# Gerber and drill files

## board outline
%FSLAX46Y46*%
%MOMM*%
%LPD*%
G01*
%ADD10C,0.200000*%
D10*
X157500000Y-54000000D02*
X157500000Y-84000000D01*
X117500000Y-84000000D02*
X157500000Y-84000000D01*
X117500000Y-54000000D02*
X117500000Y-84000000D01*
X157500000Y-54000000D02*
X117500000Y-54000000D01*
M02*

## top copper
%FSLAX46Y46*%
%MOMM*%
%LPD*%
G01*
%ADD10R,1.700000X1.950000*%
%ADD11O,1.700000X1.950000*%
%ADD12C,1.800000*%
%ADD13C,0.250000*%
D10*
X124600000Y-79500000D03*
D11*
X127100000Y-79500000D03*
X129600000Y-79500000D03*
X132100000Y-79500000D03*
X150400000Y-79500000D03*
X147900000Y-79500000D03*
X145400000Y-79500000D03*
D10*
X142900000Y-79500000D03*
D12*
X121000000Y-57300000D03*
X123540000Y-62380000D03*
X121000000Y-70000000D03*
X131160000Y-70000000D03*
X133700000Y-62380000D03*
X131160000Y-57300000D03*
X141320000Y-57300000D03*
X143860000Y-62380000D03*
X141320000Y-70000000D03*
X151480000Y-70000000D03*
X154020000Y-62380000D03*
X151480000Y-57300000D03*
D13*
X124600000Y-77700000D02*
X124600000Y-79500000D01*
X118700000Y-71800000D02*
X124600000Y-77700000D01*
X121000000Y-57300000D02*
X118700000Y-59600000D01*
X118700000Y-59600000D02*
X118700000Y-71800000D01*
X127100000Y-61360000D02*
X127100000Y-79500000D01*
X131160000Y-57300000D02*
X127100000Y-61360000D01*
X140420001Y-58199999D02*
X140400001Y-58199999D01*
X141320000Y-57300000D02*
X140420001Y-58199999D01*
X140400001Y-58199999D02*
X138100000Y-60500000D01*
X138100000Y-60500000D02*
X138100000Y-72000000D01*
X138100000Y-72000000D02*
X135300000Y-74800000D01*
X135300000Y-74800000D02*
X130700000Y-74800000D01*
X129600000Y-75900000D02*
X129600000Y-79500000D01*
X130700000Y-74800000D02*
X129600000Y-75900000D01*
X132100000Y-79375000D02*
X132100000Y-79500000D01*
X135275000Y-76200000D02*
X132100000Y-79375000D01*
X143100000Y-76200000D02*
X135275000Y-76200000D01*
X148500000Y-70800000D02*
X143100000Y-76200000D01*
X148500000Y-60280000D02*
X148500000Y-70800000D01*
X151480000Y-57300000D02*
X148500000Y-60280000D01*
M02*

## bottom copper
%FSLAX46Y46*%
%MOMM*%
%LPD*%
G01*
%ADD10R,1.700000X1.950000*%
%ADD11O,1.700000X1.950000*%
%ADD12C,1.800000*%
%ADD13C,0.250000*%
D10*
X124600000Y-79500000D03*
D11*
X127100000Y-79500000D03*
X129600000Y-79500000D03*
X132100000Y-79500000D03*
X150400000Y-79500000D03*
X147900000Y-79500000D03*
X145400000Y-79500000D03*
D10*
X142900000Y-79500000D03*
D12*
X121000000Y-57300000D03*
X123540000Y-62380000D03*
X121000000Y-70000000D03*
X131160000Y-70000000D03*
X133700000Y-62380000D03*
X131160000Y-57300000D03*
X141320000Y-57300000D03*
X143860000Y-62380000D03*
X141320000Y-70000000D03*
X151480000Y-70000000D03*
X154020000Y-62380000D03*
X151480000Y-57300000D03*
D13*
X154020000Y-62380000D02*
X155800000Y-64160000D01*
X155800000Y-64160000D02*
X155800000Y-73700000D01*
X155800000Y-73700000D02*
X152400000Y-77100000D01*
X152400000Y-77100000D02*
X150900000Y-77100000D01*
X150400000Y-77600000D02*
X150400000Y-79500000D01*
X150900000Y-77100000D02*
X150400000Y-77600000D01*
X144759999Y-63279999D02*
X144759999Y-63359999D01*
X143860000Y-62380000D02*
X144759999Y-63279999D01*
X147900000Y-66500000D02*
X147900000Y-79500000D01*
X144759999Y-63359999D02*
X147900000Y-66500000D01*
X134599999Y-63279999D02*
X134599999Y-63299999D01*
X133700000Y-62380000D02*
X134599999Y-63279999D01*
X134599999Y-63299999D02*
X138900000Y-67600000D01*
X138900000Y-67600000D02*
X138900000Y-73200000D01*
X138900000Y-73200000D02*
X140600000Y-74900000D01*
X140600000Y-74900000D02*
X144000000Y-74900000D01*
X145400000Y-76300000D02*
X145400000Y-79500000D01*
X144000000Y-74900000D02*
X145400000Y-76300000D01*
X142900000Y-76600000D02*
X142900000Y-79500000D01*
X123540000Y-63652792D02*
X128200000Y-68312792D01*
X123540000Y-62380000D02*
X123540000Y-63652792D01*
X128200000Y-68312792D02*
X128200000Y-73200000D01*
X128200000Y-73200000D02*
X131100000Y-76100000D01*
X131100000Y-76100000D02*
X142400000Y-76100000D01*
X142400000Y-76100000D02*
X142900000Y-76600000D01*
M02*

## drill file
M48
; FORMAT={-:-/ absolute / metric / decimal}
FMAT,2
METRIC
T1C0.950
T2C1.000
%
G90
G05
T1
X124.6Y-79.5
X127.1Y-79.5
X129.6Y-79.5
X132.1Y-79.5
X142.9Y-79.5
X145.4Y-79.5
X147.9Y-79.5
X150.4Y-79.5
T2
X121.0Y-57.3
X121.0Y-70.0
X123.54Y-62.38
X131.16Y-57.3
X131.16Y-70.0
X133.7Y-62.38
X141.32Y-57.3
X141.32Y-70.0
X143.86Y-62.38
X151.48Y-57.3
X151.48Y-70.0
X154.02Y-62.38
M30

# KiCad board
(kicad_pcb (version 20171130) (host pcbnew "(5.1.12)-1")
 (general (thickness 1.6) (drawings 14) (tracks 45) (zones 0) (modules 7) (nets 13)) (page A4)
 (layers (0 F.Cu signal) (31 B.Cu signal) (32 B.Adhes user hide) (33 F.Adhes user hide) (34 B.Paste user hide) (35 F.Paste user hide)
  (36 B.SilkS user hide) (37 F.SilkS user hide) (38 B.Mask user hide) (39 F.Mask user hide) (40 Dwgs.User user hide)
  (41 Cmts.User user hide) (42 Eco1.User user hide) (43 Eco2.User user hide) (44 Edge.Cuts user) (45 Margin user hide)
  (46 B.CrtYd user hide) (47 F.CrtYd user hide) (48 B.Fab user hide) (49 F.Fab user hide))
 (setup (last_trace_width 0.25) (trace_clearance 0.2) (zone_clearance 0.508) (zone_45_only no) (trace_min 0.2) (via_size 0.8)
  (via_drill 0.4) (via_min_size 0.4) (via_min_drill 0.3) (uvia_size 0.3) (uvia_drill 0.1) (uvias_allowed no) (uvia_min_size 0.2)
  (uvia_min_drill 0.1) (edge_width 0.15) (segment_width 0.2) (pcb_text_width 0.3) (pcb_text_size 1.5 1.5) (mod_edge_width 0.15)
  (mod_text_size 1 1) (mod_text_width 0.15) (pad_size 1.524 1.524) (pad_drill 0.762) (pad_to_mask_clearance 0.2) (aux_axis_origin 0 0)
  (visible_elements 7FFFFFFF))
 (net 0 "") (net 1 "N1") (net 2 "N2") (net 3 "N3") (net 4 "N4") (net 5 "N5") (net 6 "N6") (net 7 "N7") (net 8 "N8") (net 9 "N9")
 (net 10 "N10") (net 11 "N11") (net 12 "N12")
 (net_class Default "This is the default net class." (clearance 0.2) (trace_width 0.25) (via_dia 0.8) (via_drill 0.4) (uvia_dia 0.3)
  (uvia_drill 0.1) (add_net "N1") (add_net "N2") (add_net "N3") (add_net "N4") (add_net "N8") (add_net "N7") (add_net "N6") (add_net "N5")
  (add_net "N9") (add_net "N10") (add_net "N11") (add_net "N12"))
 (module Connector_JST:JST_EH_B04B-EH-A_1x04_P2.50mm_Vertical (layer F.Cu) (at 124.6 79.5)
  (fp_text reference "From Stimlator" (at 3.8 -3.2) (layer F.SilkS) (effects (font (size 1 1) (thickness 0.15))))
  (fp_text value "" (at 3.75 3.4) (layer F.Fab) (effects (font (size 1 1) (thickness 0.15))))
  (pad 1 thru_hole rect (at 0 0) (size 1.7 1.95) (drill 0.95) (layers *.Cu *.Mask) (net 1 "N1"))
  (pad 2 thru_hole oval (at 2.5 0) (size 1.7 1.95) (drill 0.95) (layers *.Cu *.Mask) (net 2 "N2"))
  (pad 3 thru_hole oval (at 5 0) (size 1.7 1.95) (drill 0.95) (layers *.Cu *.Mask) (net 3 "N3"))
  (pad 4 thru_hole oval (at 7.5 0) (size 1.7 1.95) (drill 0.95) (layers *.Cu *.Mask) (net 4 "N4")))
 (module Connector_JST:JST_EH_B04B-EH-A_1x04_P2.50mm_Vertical (layer F.Cu) (at 142.9 79.5)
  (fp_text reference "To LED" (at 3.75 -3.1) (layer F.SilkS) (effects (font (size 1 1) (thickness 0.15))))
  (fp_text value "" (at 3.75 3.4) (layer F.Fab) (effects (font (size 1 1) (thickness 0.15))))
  (pad 4 thru_hole oval (at 7.5 0) (size 1.7 1.95) (drill 0.95) (layers *.Cu *.Mask) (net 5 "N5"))
  (pad 3 thru_hole oval (at 5 0) (size 1.7 1.95) (drill 0.95) (layers *.Cu *.Mask) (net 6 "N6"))
  (pad 2 thru_hole oval (at 2.5 0) (size 1.7 1.95) (drill 0.95) (layers *.Cu *.Mask) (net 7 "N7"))
  (pad 1 thru_hole rect (at 0 0) (size 1.7 1.95) (drill 0.95) (layers *.Cu *.Mask) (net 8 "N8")))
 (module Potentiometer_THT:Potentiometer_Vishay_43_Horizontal (layer F.Cu) (at 121 70 270)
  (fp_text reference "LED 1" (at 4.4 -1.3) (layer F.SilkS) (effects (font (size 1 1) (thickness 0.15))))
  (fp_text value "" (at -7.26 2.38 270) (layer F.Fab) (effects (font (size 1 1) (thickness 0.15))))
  (pad 3 thru_hole circle (at -12.7 0 270) (size 1.8 1.8) (drill 1) (layers *.Cu *.Mask) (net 1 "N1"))
  (pad 2 thru_hole circle (at -7.62 -2.54 270) (size 1.8 1.8) (drill 1) (layers *.Cu *.Mask) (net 8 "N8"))
  (pad 1 thru_hole circle (at 0 0 270) (size 1.8 1.8) (drill 1) (layers *.Cu *.Mask) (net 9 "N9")))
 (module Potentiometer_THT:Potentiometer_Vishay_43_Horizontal (layer F.Cu) (at 131.16 70 270)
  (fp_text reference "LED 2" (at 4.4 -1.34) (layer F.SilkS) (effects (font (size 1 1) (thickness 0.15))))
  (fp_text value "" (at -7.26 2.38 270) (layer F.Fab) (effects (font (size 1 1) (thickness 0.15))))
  (pad 1 thru_hole circle (at 0 0 270) (size 1.8 1.8) (drill 1) (layers *.Cu *.Mask) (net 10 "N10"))
  (pad 2 thru_hole circle (at -7.62 -2.54 270) (size 1.8 1.8) (drill 1) (layers *.Cu *.Mask) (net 7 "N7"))
  (pad 3 thru_hole circle (at -12.7 0 270) (size 1.8 1.8) (drill 1) (layers *.Cu *.Mask) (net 2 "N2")))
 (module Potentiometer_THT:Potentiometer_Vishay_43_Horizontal (layer F.Cu) (at 141.32 70 270)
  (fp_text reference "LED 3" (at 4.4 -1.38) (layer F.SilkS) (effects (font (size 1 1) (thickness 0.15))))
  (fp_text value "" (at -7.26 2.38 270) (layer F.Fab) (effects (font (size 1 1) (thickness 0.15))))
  (pad 3 thru_hole circle (at -12.7 0 270) (size 1.8 1.8) (drill 1) (layers *.Cu *.Mask) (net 3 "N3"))
  (pad 2 thru_hole circle (at -7.62 -2.54 270) (size 1.8 1.8) (drill 1) (layers *.Cu *.Mask) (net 6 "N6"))
  (pad 1 thru_hole circle (at 0 0 270) (size 1.8 1.8) (drill 1) (layers *.Cu *.Mask) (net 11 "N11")))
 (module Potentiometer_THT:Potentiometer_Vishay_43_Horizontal (layer F.Cu) (at 151.48 70 270)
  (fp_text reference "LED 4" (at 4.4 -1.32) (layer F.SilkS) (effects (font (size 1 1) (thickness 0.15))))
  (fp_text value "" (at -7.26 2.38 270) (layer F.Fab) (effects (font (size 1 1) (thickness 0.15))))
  (pad 1 thru_hole circle (at 0 0 270) (size 1.8 1.8) (drill 1) (layers *.Cu *.Mask) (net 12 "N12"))
  (pad 2 thru_hole circle (at -7.62 -2.54 270) (size 1.8 1.8) (drill 1) (layers *.Cu *.Mask) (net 5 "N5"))
  (pad 3 thru_hole circle (at -12.7 0 270) (size 1.8 1.8) (drill 1) (layers *.Cu *.Mask) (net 4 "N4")))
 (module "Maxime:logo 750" (layer B.Cu) (at 137.5 75.1 180)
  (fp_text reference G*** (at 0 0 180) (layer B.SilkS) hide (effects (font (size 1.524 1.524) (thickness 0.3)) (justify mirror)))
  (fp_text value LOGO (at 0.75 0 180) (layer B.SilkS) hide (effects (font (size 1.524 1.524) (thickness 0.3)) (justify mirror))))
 (gr_line (start 157.5 54) (end 157.5 84) (layer Edge.Cuts) (width 0.2))
 (gr_line (start 117.5 84) (end 157.5 84) (layer Edge.Cuts) (width 0.2))
 (gr_line (start 117.5 54) (end 117.5 84) (layer Edge.Cuts) (width 0.2))
 (gr_line (start 157.5 54) (end 117.5 54) (layer Edge.Cuts) (width 0.2))
 (segment (start 124.6 77.7) (end 124.6 79.5) (width 0.25) (layer F.Cu) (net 1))
 (segment (start 118.7 71.8) (end 124.6 77.7) (width 0.25) (layer F.Cu) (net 1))
 (segment (start 121 57.3) (end 118.7 59.6) (width 0.25) (layer F.Cu) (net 1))
 (segment (start 118.7 59.6) (end 118.7 71.8) (width 0.25) (layer F.Cu) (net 1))
 (segment (start 127.1 61.36) (end 127.1 79.5) (width 0.25) (layer F.Cu) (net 2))
 (segment (start 131.16 57.3) (end 127.1 61.36) (width 0.25) (layer F.Cu) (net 2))
 (segment (start 140.420001 58.199999) (end 140.400001 58.199999) (width 0.25) (layer F.Cu) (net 3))
 (segment (start 141.32 57.3) (end 140.420001 58.199999) (width 0.25) (layer F.Cu) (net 3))
 (segment (start 140.400001 58.199999) (end 138.1 60.5) (width 0.25) (layer F.Cu) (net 3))
 (segment (start 138.1 60.5) (end 138.1 72) (width 0.25) (layer F.Cu) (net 3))
 (segment (start 138.1 72) (end 135.3 74.8) (width 0.25) (layer F.Cu) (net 3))
 (segment (start 135.3 74.8) (end 130.7 74.8) (width 0.25) (layer F.Cu) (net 3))
 (segment (start 129.6 75.9) (end 129.6 79.5) (width 0.25) (layer F.Cu) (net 3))
 (segment (start 130.7 74.8) (end 129.6 75.9) (width 0.25) (layer F.Cu) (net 3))
 (segment (start 132.1 79.375) (end 132.1 79.5) (width 0.25) (layer F.Cu) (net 4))
 (segment (start 135.275 76.2) (end 132.1 79.375) (width 0.25) (layer F.Cu) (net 4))
 (segment (start 143.1 76.2) (end 135.275 76.2) (width 0.25) (layer F.Cu) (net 4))
 (segment (start 148.5 70.8) (end 143.1 76.2) (width 0.25) (layer F.Cu) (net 4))
 (segment (start 148.5 60.28) (end 148.5 70.8) (width 0.25) (layer F.Cu) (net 4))
 (segment (start 151.48 57.3) (end 148.5 60.28) (width 0.25) (layer F.Cu) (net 4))
 (segment (start 154.02 62.38) (end 155.8 64.16) (width 0.25) (layer B.Cu) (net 5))
 (segment (start 155.8 64.16) (end 155.8 73.7) (width 0.25) (layer B.Cu) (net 5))
 (segment (start 155.8 73.7) (end 152.4 77.1) (width 0.25) (layer B.Cu) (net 5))
 (segment (start 152.4 77.1) (end 150.9 77.1) (width 0.25) (layer B.Cu) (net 5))
 (segment (start 150.4 77.6) (end 150.4 79.5) (width 0.25) (layer B.Cu) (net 5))
 (segment (start 150.9 77.1) (end 150.4 77.6) (width 0.25) (layer B.Cu) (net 5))
 (segment (start 144.759999 63.279999) (end 144.759999 63.359999) (width 0.25) (layer B.Cu) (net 6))
 (segment (start 143.86 62.38) (end 144.759999 63.279999) (width 0.25) (layer B.Cu) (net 6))
 (segment (start 147.9 66.5) (end 147.9 79.5) (width 0.25) (layer B.Cu) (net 6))
 (segment (start 144.759999 63.359999) (end 147.9 66.5) (width 0.25) (layer B.Cu) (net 6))
 (segment (start 134.599999 63.279999) (end 134.599999 63.299999) (width 0.25) (layer B.Cu) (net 7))
 (segment (start 133.7 62.38) (end 134.599999 63.279999) (width 0.25) (layer B.Cu) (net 7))
 (segment (start 134.599999 63.299999) (end 138.9 67.6) (width 0.25) (layer B.Cu) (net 7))
 (segment (start 138.9 67.6) (end 138.9 73.2) (width 0.25) (layer B.Cu) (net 7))
 (segment (start 138.9 73.2) (end 140.6 74.9) (width 0.25) (layer B.Cu) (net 7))
 (segment (start 140.6 74.9) (end 144 74.9) (width 0.25) (layer B.Cu) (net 7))
 (segment (start 145.4 76.3) (end 145.4 79.5) (width 0.25) (layer B.Cu) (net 7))
 (segment (start 144 74.9) (end 145.4 76.3) (width 0.25) (layer B.Cu) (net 7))
 (segment (start 142.9 76.6) (end 142.9 79.5) (width 0.25) (layer B.Cu) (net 8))
 (segment (start 123.54 63.652792) (end 128.2 68.312792) (width 0.25) (layer B.Cu) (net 8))
 (segment (start 123.54 62.38) (end 123.54 63.652792) (width 0.25) (layer B.Cu) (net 8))
 (segment (start 128.2 68.312792) (end 128.2 73.2) (width 0.25) (layer B.Cu) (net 8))
 (segment (start 128.2 73.2) (end 131.1 76.1) (width 0.25) (layer B.Cu) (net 8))
 (segment (start 131.1 76.1) (end 142.4 76.1) (width 0.25) (layer B.Cu) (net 8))
 (segment (start 142.4 76.1) (end 142.9 76.6) (width 0.25) (layer B.Cu) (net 8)))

